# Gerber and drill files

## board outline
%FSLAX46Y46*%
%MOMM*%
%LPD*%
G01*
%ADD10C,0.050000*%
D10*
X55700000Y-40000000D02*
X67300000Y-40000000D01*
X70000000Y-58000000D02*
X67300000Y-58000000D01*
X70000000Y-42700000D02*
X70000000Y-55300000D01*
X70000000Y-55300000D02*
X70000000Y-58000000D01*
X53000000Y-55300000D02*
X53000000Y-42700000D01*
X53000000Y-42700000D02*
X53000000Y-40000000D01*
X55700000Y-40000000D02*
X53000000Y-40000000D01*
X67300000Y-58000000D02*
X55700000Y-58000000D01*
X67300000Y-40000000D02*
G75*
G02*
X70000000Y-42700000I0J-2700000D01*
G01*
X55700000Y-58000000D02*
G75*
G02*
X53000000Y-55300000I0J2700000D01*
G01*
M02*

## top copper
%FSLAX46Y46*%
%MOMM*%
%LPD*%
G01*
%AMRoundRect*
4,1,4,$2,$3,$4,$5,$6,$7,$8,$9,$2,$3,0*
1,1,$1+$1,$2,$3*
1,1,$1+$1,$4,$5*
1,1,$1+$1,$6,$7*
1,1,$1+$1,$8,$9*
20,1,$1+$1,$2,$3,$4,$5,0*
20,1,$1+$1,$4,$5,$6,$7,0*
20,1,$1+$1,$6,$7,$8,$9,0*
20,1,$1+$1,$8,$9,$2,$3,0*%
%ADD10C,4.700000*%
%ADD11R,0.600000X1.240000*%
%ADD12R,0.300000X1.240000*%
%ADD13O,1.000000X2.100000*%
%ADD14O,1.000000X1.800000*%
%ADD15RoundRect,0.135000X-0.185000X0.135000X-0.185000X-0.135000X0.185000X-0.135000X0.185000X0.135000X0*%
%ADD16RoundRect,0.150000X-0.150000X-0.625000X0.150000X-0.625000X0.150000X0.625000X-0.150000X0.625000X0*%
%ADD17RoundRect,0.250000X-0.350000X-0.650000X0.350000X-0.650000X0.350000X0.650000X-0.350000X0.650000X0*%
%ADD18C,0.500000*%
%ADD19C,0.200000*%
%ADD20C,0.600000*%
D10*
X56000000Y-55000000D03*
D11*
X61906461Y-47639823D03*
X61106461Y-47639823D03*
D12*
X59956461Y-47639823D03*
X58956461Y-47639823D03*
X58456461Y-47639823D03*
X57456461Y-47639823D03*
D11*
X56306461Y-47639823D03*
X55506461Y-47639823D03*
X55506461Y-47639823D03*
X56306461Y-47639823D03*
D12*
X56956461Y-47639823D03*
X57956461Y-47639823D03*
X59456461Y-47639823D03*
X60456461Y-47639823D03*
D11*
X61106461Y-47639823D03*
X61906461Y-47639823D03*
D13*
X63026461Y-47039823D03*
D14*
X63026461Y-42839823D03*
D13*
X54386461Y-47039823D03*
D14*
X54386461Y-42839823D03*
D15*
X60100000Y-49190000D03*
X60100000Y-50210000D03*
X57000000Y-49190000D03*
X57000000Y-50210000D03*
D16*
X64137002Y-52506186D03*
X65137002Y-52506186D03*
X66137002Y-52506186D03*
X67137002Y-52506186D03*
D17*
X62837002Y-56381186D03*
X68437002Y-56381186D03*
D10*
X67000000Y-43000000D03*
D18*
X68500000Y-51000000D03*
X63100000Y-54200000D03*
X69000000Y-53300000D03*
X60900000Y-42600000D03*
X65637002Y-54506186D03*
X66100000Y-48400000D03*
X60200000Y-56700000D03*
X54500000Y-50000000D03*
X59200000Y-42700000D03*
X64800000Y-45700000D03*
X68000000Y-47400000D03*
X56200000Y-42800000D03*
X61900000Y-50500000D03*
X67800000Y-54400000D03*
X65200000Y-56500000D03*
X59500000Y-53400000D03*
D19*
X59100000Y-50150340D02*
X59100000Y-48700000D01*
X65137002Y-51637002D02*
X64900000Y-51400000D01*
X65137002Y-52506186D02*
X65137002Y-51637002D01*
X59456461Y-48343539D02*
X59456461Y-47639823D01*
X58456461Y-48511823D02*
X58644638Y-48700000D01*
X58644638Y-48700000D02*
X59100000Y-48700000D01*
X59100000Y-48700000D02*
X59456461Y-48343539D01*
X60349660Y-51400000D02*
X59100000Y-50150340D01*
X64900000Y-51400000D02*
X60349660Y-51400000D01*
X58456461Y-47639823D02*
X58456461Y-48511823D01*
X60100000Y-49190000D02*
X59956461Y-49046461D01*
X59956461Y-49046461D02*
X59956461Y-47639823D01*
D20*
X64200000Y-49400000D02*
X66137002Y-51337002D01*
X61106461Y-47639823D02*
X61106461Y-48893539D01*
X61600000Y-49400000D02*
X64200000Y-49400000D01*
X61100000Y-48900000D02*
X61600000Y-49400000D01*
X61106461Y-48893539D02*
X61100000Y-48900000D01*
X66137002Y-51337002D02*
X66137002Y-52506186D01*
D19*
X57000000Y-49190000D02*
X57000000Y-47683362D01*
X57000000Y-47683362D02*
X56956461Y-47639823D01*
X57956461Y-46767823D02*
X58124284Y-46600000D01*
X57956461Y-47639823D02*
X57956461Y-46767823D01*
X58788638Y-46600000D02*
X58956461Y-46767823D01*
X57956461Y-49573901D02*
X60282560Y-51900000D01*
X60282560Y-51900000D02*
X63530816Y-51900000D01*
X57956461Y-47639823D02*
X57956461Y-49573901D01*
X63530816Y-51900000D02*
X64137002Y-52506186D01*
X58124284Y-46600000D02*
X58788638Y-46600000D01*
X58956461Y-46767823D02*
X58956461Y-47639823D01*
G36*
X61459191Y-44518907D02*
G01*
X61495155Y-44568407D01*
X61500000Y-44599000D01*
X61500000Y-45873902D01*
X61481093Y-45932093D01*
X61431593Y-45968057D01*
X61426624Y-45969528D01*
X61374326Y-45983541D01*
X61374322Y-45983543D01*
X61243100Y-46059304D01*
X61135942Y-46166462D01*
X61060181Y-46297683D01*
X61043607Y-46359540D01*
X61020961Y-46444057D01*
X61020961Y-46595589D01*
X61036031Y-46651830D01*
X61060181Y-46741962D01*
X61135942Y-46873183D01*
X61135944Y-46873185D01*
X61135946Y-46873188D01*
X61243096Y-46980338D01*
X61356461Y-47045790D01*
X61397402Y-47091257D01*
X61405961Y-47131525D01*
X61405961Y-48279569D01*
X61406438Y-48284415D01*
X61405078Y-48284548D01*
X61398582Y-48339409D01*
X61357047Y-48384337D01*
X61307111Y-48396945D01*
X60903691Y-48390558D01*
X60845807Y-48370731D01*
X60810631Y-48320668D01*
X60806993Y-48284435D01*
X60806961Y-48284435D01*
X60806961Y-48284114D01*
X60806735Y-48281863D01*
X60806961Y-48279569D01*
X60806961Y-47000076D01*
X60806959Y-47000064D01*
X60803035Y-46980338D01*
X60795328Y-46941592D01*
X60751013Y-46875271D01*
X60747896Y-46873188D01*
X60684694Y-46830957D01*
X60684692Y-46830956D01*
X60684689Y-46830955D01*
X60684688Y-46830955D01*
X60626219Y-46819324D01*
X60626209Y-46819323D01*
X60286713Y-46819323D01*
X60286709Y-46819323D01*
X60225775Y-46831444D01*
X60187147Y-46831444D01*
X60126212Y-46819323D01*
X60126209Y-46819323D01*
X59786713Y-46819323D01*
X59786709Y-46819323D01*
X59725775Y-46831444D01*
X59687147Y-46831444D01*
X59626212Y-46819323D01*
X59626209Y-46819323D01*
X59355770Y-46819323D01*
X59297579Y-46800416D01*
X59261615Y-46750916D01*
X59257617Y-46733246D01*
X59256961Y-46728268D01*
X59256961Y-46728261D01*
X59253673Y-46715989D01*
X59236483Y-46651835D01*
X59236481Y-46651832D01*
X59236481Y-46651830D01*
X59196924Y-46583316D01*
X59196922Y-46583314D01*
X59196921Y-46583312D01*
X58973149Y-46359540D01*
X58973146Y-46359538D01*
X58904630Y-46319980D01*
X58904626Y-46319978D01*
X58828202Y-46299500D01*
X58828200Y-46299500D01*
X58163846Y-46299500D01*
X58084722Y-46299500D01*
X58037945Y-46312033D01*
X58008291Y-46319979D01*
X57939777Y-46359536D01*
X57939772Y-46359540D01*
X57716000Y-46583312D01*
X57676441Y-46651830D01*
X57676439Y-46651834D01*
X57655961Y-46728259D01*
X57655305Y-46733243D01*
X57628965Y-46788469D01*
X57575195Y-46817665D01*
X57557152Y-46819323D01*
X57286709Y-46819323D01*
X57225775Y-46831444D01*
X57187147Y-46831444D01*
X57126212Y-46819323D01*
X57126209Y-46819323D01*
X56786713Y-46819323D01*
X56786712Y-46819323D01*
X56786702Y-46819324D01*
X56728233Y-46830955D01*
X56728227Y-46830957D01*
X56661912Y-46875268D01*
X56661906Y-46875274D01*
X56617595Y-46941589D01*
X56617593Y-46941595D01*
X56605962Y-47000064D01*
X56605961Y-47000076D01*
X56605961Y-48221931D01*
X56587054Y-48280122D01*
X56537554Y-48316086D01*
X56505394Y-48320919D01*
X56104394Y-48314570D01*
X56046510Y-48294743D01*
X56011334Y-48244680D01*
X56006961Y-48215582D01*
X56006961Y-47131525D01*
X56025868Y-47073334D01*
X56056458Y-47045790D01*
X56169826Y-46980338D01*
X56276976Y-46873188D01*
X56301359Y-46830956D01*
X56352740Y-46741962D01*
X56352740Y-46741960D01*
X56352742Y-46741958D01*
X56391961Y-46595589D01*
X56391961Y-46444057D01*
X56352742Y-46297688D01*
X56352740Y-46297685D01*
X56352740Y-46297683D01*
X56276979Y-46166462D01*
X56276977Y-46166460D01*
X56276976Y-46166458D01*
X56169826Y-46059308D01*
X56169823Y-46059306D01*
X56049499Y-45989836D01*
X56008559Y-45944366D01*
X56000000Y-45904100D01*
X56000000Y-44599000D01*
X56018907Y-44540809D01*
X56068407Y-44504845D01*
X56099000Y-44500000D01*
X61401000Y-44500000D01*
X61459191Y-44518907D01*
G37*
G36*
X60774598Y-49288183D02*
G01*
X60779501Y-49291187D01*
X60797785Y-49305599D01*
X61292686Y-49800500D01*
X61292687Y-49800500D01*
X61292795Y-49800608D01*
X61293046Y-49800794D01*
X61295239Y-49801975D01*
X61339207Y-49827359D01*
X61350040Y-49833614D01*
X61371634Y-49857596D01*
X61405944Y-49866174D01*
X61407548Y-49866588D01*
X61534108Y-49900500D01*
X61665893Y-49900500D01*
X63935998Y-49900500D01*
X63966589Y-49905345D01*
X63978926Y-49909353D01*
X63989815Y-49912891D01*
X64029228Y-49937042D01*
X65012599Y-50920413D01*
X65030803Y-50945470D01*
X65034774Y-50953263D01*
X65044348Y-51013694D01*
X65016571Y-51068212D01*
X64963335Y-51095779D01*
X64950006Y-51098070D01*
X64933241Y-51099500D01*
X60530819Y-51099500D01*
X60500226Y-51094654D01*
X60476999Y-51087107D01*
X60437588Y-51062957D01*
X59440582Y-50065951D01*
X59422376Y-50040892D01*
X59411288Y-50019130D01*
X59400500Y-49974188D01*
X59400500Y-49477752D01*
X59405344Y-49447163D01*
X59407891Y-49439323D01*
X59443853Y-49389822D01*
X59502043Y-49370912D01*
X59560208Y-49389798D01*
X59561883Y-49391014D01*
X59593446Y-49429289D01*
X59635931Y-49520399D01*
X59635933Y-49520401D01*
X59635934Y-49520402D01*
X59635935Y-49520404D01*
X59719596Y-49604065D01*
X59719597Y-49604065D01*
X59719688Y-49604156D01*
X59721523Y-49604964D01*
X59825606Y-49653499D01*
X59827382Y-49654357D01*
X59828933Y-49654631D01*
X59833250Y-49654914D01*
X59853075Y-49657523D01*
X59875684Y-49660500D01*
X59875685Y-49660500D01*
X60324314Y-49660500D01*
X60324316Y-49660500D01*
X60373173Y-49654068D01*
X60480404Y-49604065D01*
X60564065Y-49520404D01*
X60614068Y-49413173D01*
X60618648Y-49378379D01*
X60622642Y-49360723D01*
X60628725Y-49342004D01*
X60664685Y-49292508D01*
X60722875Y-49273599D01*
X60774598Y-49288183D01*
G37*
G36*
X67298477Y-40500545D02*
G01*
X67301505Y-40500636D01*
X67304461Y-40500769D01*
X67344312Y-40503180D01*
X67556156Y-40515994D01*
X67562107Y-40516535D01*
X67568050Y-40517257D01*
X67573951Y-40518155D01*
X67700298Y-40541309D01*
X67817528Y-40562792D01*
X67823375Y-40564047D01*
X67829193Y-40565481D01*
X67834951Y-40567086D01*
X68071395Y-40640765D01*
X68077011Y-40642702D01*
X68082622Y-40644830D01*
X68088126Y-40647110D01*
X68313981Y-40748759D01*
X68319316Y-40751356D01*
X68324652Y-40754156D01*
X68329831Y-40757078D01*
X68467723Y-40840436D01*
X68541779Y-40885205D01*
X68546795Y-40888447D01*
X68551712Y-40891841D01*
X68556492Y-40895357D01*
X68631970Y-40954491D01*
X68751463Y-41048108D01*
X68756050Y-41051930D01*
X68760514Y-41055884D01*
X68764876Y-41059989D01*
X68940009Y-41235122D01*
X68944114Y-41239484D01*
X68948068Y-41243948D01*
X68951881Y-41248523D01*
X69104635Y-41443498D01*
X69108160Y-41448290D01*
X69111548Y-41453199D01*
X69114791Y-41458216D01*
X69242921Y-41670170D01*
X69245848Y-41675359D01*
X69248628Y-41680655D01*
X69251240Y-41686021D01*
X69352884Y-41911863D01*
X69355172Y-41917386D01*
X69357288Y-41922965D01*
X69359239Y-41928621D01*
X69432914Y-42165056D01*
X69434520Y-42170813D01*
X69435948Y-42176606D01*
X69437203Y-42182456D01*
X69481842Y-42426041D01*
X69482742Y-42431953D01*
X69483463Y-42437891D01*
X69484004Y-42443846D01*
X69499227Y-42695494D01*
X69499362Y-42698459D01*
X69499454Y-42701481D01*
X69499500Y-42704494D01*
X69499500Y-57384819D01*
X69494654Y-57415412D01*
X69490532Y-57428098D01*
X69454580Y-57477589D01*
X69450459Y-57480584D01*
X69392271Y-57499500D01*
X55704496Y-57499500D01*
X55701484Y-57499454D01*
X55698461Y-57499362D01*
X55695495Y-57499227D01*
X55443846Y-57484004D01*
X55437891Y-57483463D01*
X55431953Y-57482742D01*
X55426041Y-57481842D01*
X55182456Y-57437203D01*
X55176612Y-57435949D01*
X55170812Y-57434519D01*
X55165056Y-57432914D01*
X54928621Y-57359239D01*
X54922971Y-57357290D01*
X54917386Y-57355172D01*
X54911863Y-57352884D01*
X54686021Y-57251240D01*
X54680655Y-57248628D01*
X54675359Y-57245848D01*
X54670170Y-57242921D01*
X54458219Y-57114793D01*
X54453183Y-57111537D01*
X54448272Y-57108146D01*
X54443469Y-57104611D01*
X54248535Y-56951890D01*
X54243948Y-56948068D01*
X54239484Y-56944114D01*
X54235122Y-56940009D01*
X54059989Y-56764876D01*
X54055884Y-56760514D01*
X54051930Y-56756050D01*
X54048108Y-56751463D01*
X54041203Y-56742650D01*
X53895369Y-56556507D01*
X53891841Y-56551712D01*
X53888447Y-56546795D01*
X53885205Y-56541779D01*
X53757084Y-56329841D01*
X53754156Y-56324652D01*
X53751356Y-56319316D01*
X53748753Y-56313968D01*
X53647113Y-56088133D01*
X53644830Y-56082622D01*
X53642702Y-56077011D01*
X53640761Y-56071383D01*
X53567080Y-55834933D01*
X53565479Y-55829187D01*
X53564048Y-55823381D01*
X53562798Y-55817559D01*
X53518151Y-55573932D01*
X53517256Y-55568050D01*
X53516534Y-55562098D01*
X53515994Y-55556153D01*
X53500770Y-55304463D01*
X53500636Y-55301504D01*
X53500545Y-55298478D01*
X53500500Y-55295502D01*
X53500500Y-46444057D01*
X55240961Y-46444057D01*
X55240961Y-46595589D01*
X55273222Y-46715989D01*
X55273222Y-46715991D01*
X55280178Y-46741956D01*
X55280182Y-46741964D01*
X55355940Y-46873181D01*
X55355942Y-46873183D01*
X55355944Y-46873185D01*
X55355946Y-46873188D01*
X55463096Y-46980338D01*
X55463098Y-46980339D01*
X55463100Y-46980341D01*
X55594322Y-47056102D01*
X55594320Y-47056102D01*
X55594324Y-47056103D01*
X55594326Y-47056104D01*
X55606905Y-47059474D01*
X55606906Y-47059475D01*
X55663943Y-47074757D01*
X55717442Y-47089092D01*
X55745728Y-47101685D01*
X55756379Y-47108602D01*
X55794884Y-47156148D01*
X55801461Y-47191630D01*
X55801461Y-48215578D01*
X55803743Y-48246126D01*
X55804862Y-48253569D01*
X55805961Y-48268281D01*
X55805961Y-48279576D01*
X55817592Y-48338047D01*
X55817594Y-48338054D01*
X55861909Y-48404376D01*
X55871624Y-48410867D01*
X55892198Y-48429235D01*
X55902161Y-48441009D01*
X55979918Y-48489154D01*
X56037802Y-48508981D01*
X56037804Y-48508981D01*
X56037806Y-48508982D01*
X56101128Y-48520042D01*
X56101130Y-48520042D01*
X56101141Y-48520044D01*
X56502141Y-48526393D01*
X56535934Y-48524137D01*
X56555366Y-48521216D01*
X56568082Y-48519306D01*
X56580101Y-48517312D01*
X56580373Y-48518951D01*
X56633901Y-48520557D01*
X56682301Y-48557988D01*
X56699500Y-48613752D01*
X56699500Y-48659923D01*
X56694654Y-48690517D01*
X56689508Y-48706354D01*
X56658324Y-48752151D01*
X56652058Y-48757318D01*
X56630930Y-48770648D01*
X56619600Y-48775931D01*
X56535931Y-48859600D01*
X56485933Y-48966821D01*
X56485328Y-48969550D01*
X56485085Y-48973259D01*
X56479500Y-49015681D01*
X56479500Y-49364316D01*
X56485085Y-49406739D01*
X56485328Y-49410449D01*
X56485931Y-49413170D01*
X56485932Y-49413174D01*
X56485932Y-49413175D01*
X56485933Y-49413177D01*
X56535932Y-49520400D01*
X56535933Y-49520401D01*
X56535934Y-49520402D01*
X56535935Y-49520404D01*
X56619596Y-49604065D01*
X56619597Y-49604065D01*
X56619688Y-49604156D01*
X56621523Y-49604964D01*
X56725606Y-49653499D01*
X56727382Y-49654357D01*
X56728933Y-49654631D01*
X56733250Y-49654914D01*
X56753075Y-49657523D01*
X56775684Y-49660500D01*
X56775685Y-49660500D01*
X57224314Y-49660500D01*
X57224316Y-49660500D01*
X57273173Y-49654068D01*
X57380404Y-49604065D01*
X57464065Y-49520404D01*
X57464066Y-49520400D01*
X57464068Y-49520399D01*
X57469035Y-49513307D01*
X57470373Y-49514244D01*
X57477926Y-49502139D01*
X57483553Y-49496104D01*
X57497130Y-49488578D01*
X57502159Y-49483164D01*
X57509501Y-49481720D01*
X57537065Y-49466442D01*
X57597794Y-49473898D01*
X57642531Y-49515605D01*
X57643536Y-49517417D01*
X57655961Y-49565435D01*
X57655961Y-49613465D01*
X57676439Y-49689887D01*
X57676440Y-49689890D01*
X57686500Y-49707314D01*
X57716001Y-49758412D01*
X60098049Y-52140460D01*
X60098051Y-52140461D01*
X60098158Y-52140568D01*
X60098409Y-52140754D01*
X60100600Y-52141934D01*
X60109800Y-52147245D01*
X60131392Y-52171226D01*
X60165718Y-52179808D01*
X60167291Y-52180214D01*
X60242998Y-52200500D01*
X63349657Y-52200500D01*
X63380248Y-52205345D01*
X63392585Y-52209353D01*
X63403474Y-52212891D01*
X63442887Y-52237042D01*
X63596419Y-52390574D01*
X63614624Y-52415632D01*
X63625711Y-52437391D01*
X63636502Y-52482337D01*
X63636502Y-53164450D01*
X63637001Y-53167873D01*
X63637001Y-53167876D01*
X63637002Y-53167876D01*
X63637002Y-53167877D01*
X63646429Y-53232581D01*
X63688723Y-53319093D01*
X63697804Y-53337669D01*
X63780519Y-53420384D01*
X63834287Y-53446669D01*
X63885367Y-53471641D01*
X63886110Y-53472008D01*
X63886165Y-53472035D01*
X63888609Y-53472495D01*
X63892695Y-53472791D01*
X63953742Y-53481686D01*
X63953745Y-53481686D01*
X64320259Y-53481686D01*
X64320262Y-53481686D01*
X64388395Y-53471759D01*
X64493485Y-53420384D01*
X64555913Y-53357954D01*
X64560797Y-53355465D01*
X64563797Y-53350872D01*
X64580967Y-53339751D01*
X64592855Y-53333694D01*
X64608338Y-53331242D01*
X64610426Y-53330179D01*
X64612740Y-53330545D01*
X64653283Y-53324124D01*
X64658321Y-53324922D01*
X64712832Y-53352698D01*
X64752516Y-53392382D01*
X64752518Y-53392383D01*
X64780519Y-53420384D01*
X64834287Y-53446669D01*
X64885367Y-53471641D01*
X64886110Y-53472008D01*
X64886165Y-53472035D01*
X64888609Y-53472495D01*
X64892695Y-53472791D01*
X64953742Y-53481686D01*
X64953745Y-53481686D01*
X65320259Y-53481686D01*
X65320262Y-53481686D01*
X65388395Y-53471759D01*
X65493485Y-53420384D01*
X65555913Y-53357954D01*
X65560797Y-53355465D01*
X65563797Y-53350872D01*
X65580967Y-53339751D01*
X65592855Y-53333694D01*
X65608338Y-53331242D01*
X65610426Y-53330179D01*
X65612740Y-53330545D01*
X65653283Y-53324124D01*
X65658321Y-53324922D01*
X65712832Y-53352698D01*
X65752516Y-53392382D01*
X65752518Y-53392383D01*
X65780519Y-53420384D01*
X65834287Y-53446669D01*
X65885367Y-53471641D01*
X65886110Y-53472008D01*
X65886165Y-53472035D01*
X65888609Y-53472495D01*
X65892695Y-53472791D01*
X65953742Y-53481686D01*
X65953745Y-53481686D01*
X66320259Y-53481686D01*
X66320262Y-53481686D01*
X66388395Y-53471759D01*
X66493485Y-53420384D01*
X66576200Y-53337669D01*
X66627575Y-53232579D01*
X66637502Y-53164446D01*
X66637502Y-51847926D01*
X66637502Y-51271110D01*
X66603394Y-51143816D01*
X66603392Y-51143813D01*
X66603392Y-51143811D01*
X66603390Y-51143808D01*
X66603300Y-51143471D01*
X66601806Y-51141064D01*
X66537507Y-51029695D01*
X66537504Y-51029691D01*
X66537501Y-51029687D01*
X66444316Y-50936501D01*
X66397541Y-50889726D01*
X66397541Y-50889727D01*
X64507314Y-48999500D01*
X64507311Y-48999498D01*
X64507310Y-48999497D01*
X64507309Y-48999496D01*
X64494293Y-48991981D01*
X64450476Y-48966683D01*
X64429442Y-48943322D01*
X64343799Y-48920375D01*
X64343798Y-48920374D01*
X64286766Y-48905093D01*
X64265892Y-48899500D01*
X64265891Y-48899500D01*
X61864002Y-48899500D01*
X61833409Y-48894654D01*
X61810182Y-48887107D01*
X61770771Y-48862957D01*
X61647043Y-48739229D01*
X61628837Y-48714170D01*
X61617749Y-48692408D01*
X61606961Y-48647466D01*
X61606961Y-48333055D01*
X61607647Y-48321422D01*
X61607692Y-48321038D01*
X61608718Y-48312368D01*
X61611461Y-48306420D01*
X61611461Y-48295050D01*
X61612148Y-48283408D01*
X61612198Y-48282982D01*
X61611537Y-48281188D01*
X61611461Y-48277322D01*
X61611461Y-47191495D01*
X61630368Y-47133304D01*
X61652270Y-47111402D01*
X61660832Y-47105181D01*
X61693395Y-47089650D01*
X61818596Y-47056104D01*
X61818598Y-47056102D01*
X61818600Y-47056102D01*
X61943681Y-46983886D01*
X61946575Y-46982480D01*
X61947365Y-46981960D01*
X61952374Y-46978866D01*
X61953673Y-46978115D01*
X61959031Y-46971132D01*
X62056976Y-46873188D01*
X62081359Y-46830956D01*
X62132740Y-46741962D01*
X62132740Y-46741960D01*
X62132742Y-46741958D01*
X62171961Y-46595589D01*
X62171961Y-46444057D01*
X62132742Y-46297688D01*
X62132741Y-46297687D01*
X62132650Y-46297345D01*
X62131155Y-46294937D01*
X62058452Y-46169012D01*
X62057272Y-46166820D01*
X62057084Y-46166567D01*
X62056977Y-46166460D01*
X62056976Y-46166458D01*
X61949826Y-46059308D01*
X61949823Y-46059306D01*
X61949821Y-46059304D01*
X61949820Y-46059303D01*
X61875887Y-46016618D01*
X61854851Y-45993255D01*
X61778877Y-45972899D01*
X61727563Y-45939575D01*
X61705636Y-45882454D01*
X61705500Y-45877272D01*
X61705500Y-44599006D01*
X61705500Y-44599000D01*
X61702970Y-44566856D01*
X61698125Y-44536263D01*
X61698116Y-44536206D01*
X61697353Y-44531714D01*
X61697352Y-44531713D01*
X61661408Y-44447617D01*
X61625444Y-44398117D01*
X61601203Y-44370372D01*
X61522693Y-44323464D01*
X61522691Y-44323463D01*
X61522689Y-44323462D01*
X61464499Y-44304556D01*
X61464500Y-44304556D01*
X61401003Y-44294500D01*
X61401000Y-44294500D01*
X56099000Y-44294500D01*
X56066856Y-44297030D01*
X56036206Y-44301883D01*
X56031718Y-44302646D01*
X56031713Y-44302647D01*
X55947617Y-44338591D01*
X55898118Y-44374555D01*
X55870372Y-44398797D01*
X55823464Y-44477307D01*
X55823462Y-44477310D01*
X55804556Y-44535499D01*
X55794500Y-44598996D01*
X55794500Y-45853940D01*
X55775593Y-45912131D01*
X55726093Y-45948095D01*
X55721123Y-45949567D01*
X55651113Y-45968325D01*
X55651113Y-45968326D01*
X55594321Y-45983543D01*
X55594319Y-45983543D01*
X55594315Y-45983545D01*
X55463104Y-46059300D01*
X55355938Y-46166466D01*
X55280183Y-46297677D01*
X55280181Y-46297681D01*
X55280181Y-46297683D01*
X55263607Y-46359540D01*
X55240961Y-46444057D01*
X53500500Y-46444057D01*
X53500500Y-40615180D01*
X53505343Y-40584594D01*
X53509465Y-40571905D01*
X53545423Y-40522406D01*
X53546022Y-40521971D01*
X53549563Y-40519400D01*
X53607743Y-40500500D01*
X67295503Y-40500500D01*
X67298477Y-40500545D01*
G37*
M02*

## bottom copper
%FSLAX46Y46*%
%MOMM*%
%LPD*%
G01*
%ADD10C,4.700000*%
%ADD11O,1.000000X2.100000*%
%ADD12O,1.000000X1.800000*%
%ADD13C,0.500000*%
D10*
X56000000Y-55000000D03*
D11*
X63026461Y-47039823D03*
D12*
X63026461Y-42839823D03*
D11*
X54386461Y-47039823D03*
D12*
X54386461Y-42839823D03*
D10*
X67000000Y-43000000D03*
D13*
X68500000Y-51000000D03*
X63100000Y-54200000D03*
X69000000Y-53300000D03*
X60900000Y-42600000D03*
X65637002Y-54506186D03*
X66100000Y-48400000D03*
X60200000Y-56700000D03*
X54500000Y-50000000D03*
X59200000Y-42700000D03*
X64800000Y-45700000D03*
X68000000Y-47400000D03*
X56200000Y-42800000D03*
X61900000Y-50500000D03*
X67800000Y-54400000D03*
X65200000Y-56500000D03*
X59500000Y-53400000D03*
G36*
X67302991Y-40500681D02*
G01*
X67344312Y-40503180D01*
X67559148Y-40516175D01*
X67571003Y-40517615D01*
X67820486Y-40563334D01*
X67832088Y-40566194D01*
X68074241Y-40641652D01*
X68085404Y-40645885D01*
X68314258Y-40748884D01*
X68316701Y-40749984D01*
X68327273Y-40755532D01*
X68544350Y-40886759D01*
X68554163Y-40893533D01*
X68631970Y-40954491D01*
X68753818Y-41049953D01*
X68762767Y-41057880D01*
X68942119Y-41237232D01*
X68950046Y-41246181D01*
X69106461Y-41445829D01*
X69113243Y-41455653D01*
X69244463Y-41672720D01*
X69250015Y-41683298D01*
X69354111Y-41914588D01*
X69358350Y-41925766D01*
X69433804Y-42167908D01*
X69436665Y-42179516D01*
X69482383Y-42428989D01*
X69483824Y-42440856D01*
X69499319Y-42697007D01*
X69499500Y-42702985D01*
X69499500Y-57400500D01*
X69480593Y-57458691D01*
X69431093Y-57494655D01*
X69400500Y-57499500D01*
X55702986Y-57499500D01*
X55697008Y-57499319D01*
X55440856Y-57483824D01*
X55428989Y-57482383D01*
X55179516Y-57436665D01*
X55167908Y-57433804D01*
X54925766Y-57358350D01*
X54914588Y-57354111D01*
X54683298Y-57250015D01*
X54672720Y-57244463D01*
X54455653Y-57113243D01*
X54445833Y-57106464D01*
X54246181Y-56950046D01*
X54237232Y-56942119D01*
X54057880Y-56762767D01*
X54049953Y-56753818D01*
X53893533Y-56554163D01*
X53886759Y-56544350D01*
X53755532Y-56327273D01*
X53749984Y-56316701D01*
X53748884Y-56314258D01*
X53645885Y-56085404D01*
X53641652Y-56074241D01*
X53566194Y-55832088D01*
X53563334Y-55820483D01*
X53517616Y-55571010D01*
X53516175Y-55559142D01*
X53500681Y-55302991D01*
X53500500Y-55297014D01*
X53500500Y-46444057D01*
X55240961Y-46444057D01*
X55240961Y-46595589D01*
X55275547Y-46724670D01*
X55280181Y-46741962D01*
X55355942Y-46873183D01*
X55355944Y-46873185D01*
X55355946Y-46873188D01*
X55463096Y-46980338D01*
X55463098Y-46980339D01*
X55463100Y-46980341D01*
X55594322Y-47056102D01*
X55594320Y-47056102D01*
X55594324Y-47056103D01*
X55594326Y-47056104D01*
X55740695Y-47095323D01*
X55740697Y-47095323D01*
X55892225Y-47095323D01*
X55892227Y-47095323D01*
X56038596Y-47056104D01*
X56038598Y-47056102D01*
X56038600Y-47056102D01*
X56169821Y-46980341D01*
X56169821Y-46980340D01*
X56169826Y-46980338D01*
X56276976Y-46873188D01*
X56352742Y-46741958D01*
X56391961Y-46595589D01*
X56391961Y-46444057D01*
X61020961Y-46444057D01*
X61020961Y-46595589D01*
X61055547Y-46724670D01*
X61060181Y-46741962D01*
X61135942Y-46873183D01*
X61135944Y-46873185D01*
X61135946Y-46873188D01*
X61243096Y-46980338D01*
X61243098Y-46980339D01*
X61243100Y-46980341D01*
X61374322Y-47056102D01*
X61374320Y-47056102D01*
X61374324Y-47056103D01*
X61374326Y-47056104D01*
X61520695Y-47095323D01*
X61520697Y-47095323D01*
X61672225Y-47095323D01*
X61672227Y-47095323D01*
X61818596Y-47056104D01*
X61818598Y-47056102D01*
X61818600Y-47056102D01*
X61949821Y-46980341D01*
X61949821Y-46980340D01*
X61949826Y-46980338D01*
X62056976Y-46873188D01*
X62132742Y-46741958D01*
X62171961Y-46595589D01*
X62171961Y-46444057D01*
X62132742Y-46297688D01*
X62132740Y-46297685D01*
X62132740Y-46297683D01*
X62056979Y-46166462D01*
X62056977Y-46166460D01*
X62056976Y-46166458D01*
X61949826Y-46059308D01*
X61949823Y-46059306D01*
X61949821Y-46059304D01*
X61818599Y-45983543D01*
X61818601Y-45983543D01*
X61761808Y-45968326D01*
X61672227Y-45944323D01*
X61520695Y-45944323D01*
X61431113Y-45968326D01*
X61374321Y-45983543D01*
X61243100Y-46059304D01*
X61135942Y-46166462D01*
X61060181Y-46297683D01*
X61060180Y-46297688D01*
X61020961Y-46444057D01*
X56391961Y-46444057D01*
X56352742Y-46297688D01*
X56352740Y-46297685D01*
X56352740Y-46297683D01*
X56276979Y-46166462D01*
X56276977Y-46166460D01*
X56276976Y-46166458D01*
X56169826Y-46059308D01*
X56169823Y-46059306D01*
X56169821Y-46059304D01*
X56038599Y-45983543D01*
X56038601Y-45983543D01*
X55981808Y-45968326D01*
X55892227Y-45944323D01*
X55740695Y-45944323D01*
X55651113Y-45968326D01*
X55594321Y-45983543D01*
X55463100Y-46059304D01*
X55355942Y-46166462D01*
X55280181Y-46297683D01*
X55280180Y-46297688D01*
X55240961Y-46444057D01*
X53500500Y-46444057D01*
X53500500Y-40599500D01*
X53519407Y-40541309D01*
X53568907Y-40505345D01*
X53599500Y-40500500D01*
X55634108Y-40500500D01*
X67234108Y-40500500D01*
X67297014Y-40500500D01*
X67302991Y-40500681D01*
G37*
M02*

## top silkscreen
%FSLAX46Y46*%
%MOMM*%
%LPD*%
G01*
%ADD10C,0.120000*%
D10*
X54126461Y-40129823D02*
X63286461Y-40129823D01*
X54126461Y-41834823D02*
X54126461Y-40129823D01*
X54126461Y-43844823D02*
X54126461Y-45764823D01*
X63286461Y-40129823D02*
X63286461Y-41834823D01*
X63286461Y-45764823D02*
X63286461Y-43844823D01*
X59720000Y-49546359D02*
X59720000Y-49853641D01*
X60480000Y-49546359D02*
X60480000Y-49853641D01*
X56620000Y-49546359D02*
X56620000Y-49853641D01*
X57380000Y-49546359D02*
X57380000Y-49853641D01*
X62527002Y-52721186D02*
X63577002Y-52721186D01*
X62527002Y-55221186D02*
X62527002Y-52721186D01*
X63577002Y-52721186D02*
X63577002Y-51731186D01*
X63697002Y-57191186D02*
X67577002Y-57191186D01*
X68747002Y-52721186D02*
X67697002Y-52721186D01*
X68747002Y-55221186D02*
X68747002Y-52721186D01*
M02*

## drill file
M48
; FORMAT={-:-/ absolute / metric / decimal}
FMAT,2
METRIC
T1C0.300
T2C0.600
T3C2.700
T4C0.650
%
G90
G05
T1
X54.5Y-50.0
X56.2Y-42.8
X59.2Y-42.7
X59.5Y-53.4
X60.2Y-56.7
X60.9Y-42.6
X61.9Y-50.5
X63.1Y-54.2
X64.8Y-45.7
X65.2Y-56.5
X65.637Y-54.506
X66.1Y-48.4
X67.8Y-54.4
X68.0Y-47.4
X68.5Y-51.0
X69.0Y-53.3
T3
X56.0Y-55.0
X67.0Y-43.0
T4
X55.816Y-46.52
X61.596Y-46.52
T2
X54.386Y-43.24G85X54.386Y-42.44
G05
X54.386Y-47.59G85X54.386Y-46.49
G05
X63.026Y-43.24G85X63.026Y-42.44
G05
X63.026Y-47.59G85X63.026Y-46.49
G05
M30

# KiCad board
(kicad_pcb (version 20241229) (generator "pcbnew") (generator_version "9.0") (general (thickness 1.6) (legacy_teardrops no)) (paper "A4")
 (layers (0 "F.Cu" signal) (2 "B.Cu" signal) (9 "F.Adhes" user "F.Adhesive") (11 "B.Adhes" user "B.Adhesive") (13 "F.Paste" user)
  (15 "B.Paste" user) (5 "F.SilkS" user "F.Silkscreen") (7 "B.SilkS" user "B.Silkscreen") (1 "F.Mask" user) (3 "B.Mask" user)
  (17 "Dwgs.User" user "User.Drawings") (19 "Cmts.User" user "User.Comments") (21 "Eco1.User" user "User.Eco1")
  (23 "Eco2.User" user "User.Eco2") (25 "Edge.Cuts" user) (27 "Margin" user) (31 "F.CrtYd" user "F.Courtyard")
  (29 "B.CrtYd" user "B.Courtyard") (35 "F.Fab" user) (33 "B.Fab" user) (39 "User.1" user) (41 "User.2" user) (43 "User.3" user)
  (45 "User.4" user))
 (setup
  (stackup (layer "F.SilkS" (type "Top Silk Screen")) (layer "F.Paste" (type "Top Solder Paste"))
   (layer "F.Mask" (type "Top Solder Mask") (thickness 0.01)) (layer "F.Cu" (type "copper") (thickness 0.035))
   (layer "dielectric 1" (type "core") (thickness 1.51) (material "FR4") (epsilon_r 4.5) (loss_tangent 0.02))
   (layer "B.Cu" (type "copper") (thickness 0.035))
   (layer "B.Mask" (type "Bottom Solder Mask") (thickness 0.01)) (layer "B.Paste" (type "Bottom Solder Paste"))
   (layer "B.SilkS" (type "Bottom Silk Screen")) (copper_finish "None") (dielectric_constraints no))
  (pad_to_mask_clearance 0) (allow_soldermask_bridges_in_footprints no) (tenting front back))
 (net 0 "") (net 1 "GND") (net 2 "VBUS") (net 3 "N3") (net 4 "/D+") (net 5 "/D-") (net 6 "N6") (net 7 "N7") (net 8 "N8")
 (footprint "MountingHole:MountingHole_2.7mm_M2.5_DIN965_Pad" (layer "F.Cu") (at 56 55)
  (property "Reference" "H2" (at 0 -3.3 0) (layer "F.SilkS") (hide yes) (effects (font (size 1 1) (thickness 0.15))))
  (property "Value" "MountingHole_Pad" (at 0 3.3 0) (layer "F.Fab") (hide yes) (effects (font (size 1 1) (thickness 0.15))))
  (pad "1" thru_hole circle (at 0 0) (size 4.7 4.7) (drill 2.7) (layers "*.Cu" "*.Mask") (remove_unused_layers no) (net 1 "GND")
   (zone_connect 2)))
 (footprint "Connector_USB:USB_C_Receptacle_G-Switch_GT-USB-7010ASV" (layer "F.Cu") (at 58.706461 43.914823 180)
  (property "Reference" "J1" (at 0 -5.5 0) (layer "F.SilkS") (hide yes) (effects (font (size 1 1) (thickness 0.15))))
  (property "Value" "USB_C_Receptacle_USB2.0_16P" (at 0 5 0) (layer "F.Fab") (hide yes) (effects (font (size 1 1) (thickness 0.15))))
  (fp_line (start 4.58 3.785) (end -4.58 3.785) (stroke (width 0.12) (type solid)) (layer "F.SilkS"))
  (fp_line (start 4.58 2.08) (end 4.58 3.785) (stroke (width 0.12) (type solid)) (layer "F.SilkS"))
  (fp_line (start 4.58 0.07) (end 4.58 -1.85) (stroke (width 0.12) (type solid)) (layer "F.SilkS"))
  (fp_line (start -4.58 3.785) (end -4.58 2.08) (stroke (width 0.12) (type solid)) (layer "F.SilkS"))
  (fp_line (start -4.58 -1.85) (end -4.58 0.07) (stroke (width 0.12) (type solid)) (layer "F.SilkS"))
  (pad "" np_thru_hole circle (at -2.89 -2.605 180) (size 0.65 0.65) (drill 0.65) (layers "*.Cu" "*.Mask"))
  (pad "" np_thru_hole circle (at 2.89 -2.605 180) (size 0.65 0.65) (drill 0.65) (layers "*.Cu" "*.Mask"))
  (pad "A1" smd rect (at -3.2 -3.725 180) (size 0.6 1.24) (layers "F.Cu" "F.Mask" "F.Paste") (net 1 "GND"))
  (pad "A4" smd rect (at -2.4 -3.725 180) (size 0.6 1.24) (layers "F.Cu" "F.Mask" "F.Paste") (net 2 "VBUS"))
  (pad "A5" smd rect (at -1.25 -3.725 180) (size 0.3 1.24) (layers "F.Cu" "F.Mask" "F.Paste") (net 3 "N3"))
  (pad "A6" smd rect (at -0.25 -3.725 180) (size 0.3 1.24) (layers "F.Cu" "F.Mask" "F.Paste") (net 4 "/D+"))
  (pad "A7" smd rect (at 0.25 -3.725 180) (size 0.3 1.24) (layers "F.Cu" "F.Mask" "F.Paste") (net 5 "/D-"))
  (pad "A8" smd rect (at 1.25 -3.725 180) (size 0.3 1.24) (layers "F.Cu" "F.Mask" "F.Paste") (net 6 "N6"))
  (pad "A9" smd rect (at 2.4 -3.725 180) (size 0.6 1.24) (layers "F.Cu" "F.Mask" "F.Paste") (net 2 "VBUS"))
  (pad "A12" smd rect (at 3.2 -3.725 180) (size 0.6 1.24) (layers "F.Cu" "F.Mask" "F.Paste") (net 1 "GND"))
  (pad "B1" smd rect (at 3.2 -3.725 180) (size 0.6 1.24) (layers "F.Cu" "F.Mask" "F.Paste") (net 1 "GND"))
  (pad "B4" smd rect (at 2.4 -3.725 180) (size 0.6 1.24) (layers "F.Cu" "F.Mask" "F.Paste") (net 2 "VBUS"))
  (pad "B5" smd rect (at 1.75 -3.725 180) (size 0.3 1.24) (layers "F.Cu" "F.Mask" "F.Paste") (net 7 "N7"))
  (pad "B6" smd rect (at 0.75 -3.725 180) (size 0.3 1.24) (layers "F.Cu" "F.Mask" "F.Paste") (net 4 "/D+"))
  (pad "B7" smd rect (at -0.75 -3.725 180) (size 0.3 1.24) (layers "F.Cu" "F.Mask" "F.Paste") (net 5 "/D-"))
  (pad "B8" smd rect (at -1.75 -3.725 180) (size 0.3 1.24) (layers "F.Cu" "F.Mask" "F.Paste") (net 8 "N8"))
  (pad "B9" smd rect (at -2.4 -3.725 180) (size 0.6 1.24) (layers "F.Cu" "F.Mask" "F.Paste") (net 2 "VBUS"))
  (pad "B12" smd rect (at -3.2 -3.725 180) (size 0.6 1.24) (layers "F.Cu" "F.Mask" "F.Paste") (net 1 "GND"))
  (pad "S1" thru_hole oval (at -4.32 -3.125 180) (size 1 2.1) (drill oval 0.6 1.7) (layers "*.Cu" "*.Mask") (remove_unused_layers no)
   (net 1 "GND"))
  (pad "S1" thru_hole oval (at -4.32 1.075 180) (size 1 1.8) (drill oval 0.6 1.4) (layers "*.Cu" "*.Mask") (remove_unused_layers no)
   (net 1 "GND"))
  (pad "S1" thru_hole oval (at 4.32 -3.125 180) (size 1 2.1) (drill oval 0.6 1.7) (layers "*.Cu" "*.Mask") (remove_unused_layers no)
   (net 1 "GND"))
  (pad "S1" thru_hole oval (at 4.32 1.075 180) (size 1 1.8) (drill oval 0.6 1.4) (layers "*.Cu" "*.Mask") (remove_unused_layers no)
   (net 1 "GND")))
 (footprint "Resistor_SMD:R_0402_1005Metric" (layer "F.Cu") (at 60.1 49.7 -90)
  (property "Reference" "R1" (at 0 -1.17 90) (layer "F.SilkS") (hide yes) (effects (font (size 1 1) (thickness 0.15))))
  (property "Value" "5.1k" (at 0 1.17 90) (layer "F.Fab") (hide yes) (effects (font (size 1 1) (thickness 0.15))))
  (fp_line (start -0.153641 0.38) (end 0.153641 0.38) (stroke (width 0.12) (type solid)) (layer "F.SilkS"))
  (fp_line (start -0.153641 -0.38) (end 0.153641 -0.38) (stroke (width 0.12) (type solid)) (layer "F.SilkS"))
  (pad "1" smd roundrect (at -0.51 0 270) (size 0.54 0.64) (layers "F.Cu" "F.Mask" "F.Paste") (roundrect_rratio 0.25) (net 3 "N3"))
  (pad "2" smd roundrect (at 0.51 0 270) (size 0.54 0.64) (layers "F.Cu" "F.Mask" "F.Paste") (roundrect_rratio 0.25) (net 1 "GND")))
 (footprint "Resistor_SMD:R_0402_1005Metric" (layer "F.Cu") (at 57 49.7 -90)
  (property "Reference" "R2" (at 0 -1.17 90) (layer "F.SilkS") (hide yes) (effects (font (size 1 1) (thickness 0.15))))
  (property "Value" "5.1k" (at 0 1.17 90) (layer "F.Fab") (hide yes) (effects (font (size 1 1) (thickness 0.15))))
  (fp_line (start -0.153641 0.38) (end 0.153641 0.38) (stroke (width 0.12) (type solid)) (layer "F.SilkS"))
  (fp_line (start -0.153641 -0.38) (end 0.153641 -0.38) (stroke (width 0.12) (type solid)) (layer "F.SilkS"))
  (pad "1" smd roundrect (at -0.51 0 270) (size 0.54 0.64) (layers "F.Cu" "F.Mask" "F.Paste") (roundrect_rratio 0.25) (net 7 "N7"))
  (pad "2" smd roundrect (at 0.51 0 270) (size 0.54 0.64) (layers "F.Cu" "F.Mask" "F.Paste") (roundrect_rratio 0.25) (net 1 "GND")))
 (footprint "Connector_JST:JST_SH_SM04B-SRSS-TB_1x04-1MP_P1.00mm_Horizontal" (layer "F.Cu") (at 65.637002 54.506186)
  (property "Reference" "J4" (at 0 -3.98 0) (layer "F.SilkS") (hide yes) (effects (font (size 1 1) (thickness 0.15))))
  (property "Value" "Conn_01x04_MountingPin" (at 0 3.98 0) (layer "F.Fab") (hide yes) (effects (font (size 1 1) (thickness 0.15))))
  (fp_line (start -3.11 -1.785) (end -2.06 -1.785) (stroke (width 0.12) (type solid)) (layer "F.SilkS"))
  (fp_line (start -3.11 0.715) (end -3.11 -1.785) (stroke (width 0.12) (type solid)) (layer "F.SilkS"))
  (fp_line (start -2.06 -1.785) (end -2.06 -2.775) (stroke (width 0.12) (type solid)) (layer "F.SilkS"))
  (fp_line (start -1.94 2.685) (end 1.94 2.685) (stroke (width 0.12) (type solid)) (layer "F.SilkS"))
  (fp_line (start 3.11 -1.785) (end 2.06 -1.785) (stroke (width 0.12) (type solid)) (layer "F.SilkS"))
  (fp_line (start 3.11 0.715) (end 3.11 -1.785) (stroke (width 0.12) (type solid)) (layer "F.SilkS"))
  (pad "1" smd roundrect (at -1.5 -2) (size 0.6 1.55) (layers "F.Cu" "F.Mask" "F.Paste") (roundrect_rratio 0.25) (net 4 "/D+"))
  (pad "2" smd roundrect (at -0.5 -2) (size 0.6 1.55) (layers "F.Cu" "F.Mask" "F.Paste") (roundrect_rratio 0.25) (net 5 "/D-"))
  (pad "3" smd roundrect (at 0.5 -2) (size 0.6 1.55) (layers "F.Cu" "F.Mask" "F.Paste") (roundrect_rratio 0.25) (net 2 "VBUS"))
  (pad "4" smd roundrect (at 1.5 -2) (size 0.6 1.55) (layers "F.Cu" "F.Mask" "F.Paste") (roundrect_rratio 0.25) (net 1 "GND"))
  (pad "MP" smd roundrect (at -2.8 1.875) (size 1.2 1.8) (layers "F.Cu" "F.Mask" "F.Paste") (roundrect_rratio 0.208333) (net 1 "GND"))
  (pad "MP" smd roundrect (at 2.8 1.875) (size 1.2 1.8) (layers "F.Cu" "F.Mask" "F.Paste") (roundrect_rratio 0.208333) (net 1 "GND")))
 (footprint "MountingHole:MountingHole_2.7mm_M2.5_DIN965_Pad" (layer "F.Cu") (at 67 43)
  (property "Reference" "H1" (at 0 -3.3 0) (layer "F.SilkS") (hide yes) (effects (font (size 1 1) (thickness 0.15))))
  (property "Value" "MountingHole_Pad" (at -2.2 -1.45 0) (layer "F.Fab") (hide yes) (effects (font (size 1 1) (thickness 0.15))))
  (pad "1" thru_hole circle (at 0 0) (size 4.7 4.7) (drill 2.7) (layers "*.Cu" "*.Mask") (remove_unused_layers no) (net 1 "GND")
   (zone_connect 2)))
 (gr_line (start 55.7 40) (end 67.3 40) (stroke (width 0.05) (type default)) (layer "Edge.Cuts"))
 (gr_line (start 70 58) (end 67.3 58) (stroke (width 0.05) (type default)) (layer "Edge.Cuts"))
 (gr_line (start 70 42.7) (end 70 55.3) (stroke (width 0.05) (type default)) (layer "Edge.Cuts"))
 (gr_line (start 70 55.3) (end 70 58) (stroke (width 0.05) (type default)) (layer "Edge.Cuts"))
 (gr_line (start 53 55.3) (end 53 42.7) (stroke (width 0.05) (type default)) (layer "Edge.Cuts"))
 (gr_line (start 53 42.7) (end 53 40) (stroke (width 0.05) (type default)) (layer "Edge.Cuts"))
 (gr_line (start 55.7 40) (end 53 40) (stroke (width 0.05) (type default)) (layer "Edge.Cuts"))
 (gr_line (start 67.3 58) (end 55.7 58) (stroke (width 0.05) (type default)) (layer "Edge.Cuts"))
 (gr_arc (start 67.3 40) (mid 69.209188 40.790812) (end 70 42.7) (stroke (width 0.05) (type default)) (layer "Edge.Cuts"))
 (gr_arc (start 55.7 58) (mid 53.790812 57.209188) (end 53 55.3) (stroke (width 0.05) (type default)) (layer "Edge.Cuts"))
 (segment (start 59.1 50.15034) (end 59.1 48.7) (width 0.2) (layer "F.Cu") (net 5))
 (segment (start 65.137002 51.637002) (end 64.9 51.4) (width 0.2) (layer "F.Cu") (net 5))
 (segment (start 65.137002 52.506186) (end 65.137002 51.637002) (width 0.2) (layer "F.Cu") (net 5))
 (segment (start 59.456461 48.343539) (end 59.456461 47.639823) (width 0.2) (layer "F.Cu") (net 5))
 (segment (start 58.456461 48.511823) (end 58.644638 48.7) (width 0.2) (layer "F.Cu") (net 5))
 (segment (start 58.644638 48.7) (end 59.1 48.7) (width 0.2) (layer "F.Cu") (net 5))
 (segment (start 59.1 48.7) (end 59.456461 48.343539) (width 0.2) (layer "F.Cu") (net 5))
 (segment (start 60.34966 51.4) (end 59.1 50.15034) (width 0.2) (layer "F.Cu") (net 5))
 (segment (start 64.9 51.4) (end 60.34966 51.4) (width 0.2) (layer "F.Cu") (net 5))
 (segment (start 58.456461 47.639823) (end 58.456461 48.511823) (width 0.2) (layer "F.Cu") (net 5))
 (segment (start 60.1 49.19) (end 59.956461 49.046461) (width 0.2) (layer "F.Cu") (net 3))
 (segment (start 59.956461 49.046461) (end 59.956461 47.639823) (width 0.2) (layer "F.Cu") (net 3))
 (via (at 68.5 51) (size 0.5) (drill 0.3) (layers "F.Cu" "B.Cu") (free yes) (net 1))
 (via (at 63.1 54.2) (size 0.5) (drill 0.3) (layers "F.Cu" "B.Cu") (free yes) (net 1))
 (via (at 69 53.3) (size 0.5) (drill 0.3) (layers "F.Cu" "B.Cu") (free yes) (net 1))
 (via (at 60.9 42.6) (size 0.5) (drill 0.3) (layers "F.Cu" "B.Cu") (free yes) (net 1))
 (via (at 65.637002 54.506186) (size 0.5) (drill 0.3) (layers "F.Cu" "B.Cu") (free yes) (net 1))
 (via (at 66.1 48.4) (size 0.5) (drill 0.3) (layers "F.Cu" "B.Cu") (free yes) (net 1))
 (via (at 60.2 56.7) (size 0.5) (drill 0.3) (layers "F.Cu" "B.Cu") (free yes) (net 1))
 (via (at 54.5 50) (size 0.5) (drill 0.3) (layers "F.Cu" "B.Cu") (free yes) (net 1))
 (via (at 59.2 42.7) (size 0.5) (drill 0.3) (layers "F.Cu" "B.Cu") (free yes) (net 1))
 (via (at 64.8 45.7) (size 0.5) (drill 0.3) (layers "F.Cu" "B.Cu") (free yes) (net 1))
 (via (at 68 47.4) (size 0.5) (drill 0.3) (layers "F.Cu" "B.Cu") (free yes) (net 1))
 (via (at 56.2 42.8) (size 0.5) (drill 0.3) (layers "F.Cu" "B.Cu") (free yes) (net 1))
 (via (at 61.9 50.5) (size 0.5) (drill 0.3) (layers "F.Cu" "B.Cu") (free yes) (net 1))
 (via (at 67.8 54.4) (size 0.5) (drill 0.3) (layers "F.Cu" "B.Cu") (free yes) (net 1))
 (via (at 65.2 56.5) (size 0.5) (drill 0.3) (layers "F.Cu" "B.Cu") (free yes) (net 1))
 (via (at 59.5 53.4) (size 0.5) (drill 0.3) (layers "F.Cu" "B.Cu") (free yes) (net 1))
 (segment (start 64.2 49.4) (end 66.137002 51.337002) (width 0.6) (layer "F.Cu") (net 2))
 (segment (start 61.106461 47.639823) (end 61.106461 48.893539) (width 0.6) (layer "F.Cu") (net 2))
 (segment (start 61.6 49.4) (end 64.2 49.4) (width 0.6) (layer "F.Cu") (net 2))
 (segment (start 61.1 48.9) (end 61.6 49.4) (width 0.6) (layer "F.Cu") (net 2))
 (segment (start 61.106461 48.893539) (end 61.1 48.9) (width 0.6) (layer "F.Cu") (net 2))
 (segment (start 66.137002 51.337002) (end 66.137002 52.506186) (width 0.6) (layer "F.Cu") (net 2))
 (segment (start 57 49.19) (end 57 47.683362) (width 0.2) (layer "F.Cu") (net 7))
 (segment (start 57 47.683362) (end 56.956461 47.639823) (width 0.2) (layer "F.Cu") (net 7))
 (segment (start 57.956461 46.767823) (end 58.124284 46.6) (width 0.2) (layer "F.Cu") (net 4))
 (segment (start 57.956461 47.639823) (end 57.956461 46.767823) (width 0.2) (layer "F.Cu") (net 4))
 (segment (start 58.788638 46.6) (end 58.956461 46.767823) (width 0.2) (layer "F.Cu") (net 4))
 (segment (start 57.956461 49.573901) (end 60.28256 51.9) (width 0.2) (layer "F.Cu") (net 4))
 (segment (start 60.28256 51.9) (end 63.530816 51.9) (width 0.2) (layer "F.Cu") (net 4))
 (segment (start 57.956461 47.639823) (end 57.956461 49.573901) (width 0.2) (layer "F.Cu") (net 4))
 (segment (start 63.530816 51.9) (end 64.137002 52.506186) (width 0.2) (layer "F.Cu") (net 4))
 (segment (start 58.124284 46.6) (end 58.788638 46.6) (width 0.2) (layer "F.Cu") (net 4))
 (segment (start 58.956461 46.767823) (end 58.956461 47.639823) (width 0.2) (layer "F.Cu") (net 4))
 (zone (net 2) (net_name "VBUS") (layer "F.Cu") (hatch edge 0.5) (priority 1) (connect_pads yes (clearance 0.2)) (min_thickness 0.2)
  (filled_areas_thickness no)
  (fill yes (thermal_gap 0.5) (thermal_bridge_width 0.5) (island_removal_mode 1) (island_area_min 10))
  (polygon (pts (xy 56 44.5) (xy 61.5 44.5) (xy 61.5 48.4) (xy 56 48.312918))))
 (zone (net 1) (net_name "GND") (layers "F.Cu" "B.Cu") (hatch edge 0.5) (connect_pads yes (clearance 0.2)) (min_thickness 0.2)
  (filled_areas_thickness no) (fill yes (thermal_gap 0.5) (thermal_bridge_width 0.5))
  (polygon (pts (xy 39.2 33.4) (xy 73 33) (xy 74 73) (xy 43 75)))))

